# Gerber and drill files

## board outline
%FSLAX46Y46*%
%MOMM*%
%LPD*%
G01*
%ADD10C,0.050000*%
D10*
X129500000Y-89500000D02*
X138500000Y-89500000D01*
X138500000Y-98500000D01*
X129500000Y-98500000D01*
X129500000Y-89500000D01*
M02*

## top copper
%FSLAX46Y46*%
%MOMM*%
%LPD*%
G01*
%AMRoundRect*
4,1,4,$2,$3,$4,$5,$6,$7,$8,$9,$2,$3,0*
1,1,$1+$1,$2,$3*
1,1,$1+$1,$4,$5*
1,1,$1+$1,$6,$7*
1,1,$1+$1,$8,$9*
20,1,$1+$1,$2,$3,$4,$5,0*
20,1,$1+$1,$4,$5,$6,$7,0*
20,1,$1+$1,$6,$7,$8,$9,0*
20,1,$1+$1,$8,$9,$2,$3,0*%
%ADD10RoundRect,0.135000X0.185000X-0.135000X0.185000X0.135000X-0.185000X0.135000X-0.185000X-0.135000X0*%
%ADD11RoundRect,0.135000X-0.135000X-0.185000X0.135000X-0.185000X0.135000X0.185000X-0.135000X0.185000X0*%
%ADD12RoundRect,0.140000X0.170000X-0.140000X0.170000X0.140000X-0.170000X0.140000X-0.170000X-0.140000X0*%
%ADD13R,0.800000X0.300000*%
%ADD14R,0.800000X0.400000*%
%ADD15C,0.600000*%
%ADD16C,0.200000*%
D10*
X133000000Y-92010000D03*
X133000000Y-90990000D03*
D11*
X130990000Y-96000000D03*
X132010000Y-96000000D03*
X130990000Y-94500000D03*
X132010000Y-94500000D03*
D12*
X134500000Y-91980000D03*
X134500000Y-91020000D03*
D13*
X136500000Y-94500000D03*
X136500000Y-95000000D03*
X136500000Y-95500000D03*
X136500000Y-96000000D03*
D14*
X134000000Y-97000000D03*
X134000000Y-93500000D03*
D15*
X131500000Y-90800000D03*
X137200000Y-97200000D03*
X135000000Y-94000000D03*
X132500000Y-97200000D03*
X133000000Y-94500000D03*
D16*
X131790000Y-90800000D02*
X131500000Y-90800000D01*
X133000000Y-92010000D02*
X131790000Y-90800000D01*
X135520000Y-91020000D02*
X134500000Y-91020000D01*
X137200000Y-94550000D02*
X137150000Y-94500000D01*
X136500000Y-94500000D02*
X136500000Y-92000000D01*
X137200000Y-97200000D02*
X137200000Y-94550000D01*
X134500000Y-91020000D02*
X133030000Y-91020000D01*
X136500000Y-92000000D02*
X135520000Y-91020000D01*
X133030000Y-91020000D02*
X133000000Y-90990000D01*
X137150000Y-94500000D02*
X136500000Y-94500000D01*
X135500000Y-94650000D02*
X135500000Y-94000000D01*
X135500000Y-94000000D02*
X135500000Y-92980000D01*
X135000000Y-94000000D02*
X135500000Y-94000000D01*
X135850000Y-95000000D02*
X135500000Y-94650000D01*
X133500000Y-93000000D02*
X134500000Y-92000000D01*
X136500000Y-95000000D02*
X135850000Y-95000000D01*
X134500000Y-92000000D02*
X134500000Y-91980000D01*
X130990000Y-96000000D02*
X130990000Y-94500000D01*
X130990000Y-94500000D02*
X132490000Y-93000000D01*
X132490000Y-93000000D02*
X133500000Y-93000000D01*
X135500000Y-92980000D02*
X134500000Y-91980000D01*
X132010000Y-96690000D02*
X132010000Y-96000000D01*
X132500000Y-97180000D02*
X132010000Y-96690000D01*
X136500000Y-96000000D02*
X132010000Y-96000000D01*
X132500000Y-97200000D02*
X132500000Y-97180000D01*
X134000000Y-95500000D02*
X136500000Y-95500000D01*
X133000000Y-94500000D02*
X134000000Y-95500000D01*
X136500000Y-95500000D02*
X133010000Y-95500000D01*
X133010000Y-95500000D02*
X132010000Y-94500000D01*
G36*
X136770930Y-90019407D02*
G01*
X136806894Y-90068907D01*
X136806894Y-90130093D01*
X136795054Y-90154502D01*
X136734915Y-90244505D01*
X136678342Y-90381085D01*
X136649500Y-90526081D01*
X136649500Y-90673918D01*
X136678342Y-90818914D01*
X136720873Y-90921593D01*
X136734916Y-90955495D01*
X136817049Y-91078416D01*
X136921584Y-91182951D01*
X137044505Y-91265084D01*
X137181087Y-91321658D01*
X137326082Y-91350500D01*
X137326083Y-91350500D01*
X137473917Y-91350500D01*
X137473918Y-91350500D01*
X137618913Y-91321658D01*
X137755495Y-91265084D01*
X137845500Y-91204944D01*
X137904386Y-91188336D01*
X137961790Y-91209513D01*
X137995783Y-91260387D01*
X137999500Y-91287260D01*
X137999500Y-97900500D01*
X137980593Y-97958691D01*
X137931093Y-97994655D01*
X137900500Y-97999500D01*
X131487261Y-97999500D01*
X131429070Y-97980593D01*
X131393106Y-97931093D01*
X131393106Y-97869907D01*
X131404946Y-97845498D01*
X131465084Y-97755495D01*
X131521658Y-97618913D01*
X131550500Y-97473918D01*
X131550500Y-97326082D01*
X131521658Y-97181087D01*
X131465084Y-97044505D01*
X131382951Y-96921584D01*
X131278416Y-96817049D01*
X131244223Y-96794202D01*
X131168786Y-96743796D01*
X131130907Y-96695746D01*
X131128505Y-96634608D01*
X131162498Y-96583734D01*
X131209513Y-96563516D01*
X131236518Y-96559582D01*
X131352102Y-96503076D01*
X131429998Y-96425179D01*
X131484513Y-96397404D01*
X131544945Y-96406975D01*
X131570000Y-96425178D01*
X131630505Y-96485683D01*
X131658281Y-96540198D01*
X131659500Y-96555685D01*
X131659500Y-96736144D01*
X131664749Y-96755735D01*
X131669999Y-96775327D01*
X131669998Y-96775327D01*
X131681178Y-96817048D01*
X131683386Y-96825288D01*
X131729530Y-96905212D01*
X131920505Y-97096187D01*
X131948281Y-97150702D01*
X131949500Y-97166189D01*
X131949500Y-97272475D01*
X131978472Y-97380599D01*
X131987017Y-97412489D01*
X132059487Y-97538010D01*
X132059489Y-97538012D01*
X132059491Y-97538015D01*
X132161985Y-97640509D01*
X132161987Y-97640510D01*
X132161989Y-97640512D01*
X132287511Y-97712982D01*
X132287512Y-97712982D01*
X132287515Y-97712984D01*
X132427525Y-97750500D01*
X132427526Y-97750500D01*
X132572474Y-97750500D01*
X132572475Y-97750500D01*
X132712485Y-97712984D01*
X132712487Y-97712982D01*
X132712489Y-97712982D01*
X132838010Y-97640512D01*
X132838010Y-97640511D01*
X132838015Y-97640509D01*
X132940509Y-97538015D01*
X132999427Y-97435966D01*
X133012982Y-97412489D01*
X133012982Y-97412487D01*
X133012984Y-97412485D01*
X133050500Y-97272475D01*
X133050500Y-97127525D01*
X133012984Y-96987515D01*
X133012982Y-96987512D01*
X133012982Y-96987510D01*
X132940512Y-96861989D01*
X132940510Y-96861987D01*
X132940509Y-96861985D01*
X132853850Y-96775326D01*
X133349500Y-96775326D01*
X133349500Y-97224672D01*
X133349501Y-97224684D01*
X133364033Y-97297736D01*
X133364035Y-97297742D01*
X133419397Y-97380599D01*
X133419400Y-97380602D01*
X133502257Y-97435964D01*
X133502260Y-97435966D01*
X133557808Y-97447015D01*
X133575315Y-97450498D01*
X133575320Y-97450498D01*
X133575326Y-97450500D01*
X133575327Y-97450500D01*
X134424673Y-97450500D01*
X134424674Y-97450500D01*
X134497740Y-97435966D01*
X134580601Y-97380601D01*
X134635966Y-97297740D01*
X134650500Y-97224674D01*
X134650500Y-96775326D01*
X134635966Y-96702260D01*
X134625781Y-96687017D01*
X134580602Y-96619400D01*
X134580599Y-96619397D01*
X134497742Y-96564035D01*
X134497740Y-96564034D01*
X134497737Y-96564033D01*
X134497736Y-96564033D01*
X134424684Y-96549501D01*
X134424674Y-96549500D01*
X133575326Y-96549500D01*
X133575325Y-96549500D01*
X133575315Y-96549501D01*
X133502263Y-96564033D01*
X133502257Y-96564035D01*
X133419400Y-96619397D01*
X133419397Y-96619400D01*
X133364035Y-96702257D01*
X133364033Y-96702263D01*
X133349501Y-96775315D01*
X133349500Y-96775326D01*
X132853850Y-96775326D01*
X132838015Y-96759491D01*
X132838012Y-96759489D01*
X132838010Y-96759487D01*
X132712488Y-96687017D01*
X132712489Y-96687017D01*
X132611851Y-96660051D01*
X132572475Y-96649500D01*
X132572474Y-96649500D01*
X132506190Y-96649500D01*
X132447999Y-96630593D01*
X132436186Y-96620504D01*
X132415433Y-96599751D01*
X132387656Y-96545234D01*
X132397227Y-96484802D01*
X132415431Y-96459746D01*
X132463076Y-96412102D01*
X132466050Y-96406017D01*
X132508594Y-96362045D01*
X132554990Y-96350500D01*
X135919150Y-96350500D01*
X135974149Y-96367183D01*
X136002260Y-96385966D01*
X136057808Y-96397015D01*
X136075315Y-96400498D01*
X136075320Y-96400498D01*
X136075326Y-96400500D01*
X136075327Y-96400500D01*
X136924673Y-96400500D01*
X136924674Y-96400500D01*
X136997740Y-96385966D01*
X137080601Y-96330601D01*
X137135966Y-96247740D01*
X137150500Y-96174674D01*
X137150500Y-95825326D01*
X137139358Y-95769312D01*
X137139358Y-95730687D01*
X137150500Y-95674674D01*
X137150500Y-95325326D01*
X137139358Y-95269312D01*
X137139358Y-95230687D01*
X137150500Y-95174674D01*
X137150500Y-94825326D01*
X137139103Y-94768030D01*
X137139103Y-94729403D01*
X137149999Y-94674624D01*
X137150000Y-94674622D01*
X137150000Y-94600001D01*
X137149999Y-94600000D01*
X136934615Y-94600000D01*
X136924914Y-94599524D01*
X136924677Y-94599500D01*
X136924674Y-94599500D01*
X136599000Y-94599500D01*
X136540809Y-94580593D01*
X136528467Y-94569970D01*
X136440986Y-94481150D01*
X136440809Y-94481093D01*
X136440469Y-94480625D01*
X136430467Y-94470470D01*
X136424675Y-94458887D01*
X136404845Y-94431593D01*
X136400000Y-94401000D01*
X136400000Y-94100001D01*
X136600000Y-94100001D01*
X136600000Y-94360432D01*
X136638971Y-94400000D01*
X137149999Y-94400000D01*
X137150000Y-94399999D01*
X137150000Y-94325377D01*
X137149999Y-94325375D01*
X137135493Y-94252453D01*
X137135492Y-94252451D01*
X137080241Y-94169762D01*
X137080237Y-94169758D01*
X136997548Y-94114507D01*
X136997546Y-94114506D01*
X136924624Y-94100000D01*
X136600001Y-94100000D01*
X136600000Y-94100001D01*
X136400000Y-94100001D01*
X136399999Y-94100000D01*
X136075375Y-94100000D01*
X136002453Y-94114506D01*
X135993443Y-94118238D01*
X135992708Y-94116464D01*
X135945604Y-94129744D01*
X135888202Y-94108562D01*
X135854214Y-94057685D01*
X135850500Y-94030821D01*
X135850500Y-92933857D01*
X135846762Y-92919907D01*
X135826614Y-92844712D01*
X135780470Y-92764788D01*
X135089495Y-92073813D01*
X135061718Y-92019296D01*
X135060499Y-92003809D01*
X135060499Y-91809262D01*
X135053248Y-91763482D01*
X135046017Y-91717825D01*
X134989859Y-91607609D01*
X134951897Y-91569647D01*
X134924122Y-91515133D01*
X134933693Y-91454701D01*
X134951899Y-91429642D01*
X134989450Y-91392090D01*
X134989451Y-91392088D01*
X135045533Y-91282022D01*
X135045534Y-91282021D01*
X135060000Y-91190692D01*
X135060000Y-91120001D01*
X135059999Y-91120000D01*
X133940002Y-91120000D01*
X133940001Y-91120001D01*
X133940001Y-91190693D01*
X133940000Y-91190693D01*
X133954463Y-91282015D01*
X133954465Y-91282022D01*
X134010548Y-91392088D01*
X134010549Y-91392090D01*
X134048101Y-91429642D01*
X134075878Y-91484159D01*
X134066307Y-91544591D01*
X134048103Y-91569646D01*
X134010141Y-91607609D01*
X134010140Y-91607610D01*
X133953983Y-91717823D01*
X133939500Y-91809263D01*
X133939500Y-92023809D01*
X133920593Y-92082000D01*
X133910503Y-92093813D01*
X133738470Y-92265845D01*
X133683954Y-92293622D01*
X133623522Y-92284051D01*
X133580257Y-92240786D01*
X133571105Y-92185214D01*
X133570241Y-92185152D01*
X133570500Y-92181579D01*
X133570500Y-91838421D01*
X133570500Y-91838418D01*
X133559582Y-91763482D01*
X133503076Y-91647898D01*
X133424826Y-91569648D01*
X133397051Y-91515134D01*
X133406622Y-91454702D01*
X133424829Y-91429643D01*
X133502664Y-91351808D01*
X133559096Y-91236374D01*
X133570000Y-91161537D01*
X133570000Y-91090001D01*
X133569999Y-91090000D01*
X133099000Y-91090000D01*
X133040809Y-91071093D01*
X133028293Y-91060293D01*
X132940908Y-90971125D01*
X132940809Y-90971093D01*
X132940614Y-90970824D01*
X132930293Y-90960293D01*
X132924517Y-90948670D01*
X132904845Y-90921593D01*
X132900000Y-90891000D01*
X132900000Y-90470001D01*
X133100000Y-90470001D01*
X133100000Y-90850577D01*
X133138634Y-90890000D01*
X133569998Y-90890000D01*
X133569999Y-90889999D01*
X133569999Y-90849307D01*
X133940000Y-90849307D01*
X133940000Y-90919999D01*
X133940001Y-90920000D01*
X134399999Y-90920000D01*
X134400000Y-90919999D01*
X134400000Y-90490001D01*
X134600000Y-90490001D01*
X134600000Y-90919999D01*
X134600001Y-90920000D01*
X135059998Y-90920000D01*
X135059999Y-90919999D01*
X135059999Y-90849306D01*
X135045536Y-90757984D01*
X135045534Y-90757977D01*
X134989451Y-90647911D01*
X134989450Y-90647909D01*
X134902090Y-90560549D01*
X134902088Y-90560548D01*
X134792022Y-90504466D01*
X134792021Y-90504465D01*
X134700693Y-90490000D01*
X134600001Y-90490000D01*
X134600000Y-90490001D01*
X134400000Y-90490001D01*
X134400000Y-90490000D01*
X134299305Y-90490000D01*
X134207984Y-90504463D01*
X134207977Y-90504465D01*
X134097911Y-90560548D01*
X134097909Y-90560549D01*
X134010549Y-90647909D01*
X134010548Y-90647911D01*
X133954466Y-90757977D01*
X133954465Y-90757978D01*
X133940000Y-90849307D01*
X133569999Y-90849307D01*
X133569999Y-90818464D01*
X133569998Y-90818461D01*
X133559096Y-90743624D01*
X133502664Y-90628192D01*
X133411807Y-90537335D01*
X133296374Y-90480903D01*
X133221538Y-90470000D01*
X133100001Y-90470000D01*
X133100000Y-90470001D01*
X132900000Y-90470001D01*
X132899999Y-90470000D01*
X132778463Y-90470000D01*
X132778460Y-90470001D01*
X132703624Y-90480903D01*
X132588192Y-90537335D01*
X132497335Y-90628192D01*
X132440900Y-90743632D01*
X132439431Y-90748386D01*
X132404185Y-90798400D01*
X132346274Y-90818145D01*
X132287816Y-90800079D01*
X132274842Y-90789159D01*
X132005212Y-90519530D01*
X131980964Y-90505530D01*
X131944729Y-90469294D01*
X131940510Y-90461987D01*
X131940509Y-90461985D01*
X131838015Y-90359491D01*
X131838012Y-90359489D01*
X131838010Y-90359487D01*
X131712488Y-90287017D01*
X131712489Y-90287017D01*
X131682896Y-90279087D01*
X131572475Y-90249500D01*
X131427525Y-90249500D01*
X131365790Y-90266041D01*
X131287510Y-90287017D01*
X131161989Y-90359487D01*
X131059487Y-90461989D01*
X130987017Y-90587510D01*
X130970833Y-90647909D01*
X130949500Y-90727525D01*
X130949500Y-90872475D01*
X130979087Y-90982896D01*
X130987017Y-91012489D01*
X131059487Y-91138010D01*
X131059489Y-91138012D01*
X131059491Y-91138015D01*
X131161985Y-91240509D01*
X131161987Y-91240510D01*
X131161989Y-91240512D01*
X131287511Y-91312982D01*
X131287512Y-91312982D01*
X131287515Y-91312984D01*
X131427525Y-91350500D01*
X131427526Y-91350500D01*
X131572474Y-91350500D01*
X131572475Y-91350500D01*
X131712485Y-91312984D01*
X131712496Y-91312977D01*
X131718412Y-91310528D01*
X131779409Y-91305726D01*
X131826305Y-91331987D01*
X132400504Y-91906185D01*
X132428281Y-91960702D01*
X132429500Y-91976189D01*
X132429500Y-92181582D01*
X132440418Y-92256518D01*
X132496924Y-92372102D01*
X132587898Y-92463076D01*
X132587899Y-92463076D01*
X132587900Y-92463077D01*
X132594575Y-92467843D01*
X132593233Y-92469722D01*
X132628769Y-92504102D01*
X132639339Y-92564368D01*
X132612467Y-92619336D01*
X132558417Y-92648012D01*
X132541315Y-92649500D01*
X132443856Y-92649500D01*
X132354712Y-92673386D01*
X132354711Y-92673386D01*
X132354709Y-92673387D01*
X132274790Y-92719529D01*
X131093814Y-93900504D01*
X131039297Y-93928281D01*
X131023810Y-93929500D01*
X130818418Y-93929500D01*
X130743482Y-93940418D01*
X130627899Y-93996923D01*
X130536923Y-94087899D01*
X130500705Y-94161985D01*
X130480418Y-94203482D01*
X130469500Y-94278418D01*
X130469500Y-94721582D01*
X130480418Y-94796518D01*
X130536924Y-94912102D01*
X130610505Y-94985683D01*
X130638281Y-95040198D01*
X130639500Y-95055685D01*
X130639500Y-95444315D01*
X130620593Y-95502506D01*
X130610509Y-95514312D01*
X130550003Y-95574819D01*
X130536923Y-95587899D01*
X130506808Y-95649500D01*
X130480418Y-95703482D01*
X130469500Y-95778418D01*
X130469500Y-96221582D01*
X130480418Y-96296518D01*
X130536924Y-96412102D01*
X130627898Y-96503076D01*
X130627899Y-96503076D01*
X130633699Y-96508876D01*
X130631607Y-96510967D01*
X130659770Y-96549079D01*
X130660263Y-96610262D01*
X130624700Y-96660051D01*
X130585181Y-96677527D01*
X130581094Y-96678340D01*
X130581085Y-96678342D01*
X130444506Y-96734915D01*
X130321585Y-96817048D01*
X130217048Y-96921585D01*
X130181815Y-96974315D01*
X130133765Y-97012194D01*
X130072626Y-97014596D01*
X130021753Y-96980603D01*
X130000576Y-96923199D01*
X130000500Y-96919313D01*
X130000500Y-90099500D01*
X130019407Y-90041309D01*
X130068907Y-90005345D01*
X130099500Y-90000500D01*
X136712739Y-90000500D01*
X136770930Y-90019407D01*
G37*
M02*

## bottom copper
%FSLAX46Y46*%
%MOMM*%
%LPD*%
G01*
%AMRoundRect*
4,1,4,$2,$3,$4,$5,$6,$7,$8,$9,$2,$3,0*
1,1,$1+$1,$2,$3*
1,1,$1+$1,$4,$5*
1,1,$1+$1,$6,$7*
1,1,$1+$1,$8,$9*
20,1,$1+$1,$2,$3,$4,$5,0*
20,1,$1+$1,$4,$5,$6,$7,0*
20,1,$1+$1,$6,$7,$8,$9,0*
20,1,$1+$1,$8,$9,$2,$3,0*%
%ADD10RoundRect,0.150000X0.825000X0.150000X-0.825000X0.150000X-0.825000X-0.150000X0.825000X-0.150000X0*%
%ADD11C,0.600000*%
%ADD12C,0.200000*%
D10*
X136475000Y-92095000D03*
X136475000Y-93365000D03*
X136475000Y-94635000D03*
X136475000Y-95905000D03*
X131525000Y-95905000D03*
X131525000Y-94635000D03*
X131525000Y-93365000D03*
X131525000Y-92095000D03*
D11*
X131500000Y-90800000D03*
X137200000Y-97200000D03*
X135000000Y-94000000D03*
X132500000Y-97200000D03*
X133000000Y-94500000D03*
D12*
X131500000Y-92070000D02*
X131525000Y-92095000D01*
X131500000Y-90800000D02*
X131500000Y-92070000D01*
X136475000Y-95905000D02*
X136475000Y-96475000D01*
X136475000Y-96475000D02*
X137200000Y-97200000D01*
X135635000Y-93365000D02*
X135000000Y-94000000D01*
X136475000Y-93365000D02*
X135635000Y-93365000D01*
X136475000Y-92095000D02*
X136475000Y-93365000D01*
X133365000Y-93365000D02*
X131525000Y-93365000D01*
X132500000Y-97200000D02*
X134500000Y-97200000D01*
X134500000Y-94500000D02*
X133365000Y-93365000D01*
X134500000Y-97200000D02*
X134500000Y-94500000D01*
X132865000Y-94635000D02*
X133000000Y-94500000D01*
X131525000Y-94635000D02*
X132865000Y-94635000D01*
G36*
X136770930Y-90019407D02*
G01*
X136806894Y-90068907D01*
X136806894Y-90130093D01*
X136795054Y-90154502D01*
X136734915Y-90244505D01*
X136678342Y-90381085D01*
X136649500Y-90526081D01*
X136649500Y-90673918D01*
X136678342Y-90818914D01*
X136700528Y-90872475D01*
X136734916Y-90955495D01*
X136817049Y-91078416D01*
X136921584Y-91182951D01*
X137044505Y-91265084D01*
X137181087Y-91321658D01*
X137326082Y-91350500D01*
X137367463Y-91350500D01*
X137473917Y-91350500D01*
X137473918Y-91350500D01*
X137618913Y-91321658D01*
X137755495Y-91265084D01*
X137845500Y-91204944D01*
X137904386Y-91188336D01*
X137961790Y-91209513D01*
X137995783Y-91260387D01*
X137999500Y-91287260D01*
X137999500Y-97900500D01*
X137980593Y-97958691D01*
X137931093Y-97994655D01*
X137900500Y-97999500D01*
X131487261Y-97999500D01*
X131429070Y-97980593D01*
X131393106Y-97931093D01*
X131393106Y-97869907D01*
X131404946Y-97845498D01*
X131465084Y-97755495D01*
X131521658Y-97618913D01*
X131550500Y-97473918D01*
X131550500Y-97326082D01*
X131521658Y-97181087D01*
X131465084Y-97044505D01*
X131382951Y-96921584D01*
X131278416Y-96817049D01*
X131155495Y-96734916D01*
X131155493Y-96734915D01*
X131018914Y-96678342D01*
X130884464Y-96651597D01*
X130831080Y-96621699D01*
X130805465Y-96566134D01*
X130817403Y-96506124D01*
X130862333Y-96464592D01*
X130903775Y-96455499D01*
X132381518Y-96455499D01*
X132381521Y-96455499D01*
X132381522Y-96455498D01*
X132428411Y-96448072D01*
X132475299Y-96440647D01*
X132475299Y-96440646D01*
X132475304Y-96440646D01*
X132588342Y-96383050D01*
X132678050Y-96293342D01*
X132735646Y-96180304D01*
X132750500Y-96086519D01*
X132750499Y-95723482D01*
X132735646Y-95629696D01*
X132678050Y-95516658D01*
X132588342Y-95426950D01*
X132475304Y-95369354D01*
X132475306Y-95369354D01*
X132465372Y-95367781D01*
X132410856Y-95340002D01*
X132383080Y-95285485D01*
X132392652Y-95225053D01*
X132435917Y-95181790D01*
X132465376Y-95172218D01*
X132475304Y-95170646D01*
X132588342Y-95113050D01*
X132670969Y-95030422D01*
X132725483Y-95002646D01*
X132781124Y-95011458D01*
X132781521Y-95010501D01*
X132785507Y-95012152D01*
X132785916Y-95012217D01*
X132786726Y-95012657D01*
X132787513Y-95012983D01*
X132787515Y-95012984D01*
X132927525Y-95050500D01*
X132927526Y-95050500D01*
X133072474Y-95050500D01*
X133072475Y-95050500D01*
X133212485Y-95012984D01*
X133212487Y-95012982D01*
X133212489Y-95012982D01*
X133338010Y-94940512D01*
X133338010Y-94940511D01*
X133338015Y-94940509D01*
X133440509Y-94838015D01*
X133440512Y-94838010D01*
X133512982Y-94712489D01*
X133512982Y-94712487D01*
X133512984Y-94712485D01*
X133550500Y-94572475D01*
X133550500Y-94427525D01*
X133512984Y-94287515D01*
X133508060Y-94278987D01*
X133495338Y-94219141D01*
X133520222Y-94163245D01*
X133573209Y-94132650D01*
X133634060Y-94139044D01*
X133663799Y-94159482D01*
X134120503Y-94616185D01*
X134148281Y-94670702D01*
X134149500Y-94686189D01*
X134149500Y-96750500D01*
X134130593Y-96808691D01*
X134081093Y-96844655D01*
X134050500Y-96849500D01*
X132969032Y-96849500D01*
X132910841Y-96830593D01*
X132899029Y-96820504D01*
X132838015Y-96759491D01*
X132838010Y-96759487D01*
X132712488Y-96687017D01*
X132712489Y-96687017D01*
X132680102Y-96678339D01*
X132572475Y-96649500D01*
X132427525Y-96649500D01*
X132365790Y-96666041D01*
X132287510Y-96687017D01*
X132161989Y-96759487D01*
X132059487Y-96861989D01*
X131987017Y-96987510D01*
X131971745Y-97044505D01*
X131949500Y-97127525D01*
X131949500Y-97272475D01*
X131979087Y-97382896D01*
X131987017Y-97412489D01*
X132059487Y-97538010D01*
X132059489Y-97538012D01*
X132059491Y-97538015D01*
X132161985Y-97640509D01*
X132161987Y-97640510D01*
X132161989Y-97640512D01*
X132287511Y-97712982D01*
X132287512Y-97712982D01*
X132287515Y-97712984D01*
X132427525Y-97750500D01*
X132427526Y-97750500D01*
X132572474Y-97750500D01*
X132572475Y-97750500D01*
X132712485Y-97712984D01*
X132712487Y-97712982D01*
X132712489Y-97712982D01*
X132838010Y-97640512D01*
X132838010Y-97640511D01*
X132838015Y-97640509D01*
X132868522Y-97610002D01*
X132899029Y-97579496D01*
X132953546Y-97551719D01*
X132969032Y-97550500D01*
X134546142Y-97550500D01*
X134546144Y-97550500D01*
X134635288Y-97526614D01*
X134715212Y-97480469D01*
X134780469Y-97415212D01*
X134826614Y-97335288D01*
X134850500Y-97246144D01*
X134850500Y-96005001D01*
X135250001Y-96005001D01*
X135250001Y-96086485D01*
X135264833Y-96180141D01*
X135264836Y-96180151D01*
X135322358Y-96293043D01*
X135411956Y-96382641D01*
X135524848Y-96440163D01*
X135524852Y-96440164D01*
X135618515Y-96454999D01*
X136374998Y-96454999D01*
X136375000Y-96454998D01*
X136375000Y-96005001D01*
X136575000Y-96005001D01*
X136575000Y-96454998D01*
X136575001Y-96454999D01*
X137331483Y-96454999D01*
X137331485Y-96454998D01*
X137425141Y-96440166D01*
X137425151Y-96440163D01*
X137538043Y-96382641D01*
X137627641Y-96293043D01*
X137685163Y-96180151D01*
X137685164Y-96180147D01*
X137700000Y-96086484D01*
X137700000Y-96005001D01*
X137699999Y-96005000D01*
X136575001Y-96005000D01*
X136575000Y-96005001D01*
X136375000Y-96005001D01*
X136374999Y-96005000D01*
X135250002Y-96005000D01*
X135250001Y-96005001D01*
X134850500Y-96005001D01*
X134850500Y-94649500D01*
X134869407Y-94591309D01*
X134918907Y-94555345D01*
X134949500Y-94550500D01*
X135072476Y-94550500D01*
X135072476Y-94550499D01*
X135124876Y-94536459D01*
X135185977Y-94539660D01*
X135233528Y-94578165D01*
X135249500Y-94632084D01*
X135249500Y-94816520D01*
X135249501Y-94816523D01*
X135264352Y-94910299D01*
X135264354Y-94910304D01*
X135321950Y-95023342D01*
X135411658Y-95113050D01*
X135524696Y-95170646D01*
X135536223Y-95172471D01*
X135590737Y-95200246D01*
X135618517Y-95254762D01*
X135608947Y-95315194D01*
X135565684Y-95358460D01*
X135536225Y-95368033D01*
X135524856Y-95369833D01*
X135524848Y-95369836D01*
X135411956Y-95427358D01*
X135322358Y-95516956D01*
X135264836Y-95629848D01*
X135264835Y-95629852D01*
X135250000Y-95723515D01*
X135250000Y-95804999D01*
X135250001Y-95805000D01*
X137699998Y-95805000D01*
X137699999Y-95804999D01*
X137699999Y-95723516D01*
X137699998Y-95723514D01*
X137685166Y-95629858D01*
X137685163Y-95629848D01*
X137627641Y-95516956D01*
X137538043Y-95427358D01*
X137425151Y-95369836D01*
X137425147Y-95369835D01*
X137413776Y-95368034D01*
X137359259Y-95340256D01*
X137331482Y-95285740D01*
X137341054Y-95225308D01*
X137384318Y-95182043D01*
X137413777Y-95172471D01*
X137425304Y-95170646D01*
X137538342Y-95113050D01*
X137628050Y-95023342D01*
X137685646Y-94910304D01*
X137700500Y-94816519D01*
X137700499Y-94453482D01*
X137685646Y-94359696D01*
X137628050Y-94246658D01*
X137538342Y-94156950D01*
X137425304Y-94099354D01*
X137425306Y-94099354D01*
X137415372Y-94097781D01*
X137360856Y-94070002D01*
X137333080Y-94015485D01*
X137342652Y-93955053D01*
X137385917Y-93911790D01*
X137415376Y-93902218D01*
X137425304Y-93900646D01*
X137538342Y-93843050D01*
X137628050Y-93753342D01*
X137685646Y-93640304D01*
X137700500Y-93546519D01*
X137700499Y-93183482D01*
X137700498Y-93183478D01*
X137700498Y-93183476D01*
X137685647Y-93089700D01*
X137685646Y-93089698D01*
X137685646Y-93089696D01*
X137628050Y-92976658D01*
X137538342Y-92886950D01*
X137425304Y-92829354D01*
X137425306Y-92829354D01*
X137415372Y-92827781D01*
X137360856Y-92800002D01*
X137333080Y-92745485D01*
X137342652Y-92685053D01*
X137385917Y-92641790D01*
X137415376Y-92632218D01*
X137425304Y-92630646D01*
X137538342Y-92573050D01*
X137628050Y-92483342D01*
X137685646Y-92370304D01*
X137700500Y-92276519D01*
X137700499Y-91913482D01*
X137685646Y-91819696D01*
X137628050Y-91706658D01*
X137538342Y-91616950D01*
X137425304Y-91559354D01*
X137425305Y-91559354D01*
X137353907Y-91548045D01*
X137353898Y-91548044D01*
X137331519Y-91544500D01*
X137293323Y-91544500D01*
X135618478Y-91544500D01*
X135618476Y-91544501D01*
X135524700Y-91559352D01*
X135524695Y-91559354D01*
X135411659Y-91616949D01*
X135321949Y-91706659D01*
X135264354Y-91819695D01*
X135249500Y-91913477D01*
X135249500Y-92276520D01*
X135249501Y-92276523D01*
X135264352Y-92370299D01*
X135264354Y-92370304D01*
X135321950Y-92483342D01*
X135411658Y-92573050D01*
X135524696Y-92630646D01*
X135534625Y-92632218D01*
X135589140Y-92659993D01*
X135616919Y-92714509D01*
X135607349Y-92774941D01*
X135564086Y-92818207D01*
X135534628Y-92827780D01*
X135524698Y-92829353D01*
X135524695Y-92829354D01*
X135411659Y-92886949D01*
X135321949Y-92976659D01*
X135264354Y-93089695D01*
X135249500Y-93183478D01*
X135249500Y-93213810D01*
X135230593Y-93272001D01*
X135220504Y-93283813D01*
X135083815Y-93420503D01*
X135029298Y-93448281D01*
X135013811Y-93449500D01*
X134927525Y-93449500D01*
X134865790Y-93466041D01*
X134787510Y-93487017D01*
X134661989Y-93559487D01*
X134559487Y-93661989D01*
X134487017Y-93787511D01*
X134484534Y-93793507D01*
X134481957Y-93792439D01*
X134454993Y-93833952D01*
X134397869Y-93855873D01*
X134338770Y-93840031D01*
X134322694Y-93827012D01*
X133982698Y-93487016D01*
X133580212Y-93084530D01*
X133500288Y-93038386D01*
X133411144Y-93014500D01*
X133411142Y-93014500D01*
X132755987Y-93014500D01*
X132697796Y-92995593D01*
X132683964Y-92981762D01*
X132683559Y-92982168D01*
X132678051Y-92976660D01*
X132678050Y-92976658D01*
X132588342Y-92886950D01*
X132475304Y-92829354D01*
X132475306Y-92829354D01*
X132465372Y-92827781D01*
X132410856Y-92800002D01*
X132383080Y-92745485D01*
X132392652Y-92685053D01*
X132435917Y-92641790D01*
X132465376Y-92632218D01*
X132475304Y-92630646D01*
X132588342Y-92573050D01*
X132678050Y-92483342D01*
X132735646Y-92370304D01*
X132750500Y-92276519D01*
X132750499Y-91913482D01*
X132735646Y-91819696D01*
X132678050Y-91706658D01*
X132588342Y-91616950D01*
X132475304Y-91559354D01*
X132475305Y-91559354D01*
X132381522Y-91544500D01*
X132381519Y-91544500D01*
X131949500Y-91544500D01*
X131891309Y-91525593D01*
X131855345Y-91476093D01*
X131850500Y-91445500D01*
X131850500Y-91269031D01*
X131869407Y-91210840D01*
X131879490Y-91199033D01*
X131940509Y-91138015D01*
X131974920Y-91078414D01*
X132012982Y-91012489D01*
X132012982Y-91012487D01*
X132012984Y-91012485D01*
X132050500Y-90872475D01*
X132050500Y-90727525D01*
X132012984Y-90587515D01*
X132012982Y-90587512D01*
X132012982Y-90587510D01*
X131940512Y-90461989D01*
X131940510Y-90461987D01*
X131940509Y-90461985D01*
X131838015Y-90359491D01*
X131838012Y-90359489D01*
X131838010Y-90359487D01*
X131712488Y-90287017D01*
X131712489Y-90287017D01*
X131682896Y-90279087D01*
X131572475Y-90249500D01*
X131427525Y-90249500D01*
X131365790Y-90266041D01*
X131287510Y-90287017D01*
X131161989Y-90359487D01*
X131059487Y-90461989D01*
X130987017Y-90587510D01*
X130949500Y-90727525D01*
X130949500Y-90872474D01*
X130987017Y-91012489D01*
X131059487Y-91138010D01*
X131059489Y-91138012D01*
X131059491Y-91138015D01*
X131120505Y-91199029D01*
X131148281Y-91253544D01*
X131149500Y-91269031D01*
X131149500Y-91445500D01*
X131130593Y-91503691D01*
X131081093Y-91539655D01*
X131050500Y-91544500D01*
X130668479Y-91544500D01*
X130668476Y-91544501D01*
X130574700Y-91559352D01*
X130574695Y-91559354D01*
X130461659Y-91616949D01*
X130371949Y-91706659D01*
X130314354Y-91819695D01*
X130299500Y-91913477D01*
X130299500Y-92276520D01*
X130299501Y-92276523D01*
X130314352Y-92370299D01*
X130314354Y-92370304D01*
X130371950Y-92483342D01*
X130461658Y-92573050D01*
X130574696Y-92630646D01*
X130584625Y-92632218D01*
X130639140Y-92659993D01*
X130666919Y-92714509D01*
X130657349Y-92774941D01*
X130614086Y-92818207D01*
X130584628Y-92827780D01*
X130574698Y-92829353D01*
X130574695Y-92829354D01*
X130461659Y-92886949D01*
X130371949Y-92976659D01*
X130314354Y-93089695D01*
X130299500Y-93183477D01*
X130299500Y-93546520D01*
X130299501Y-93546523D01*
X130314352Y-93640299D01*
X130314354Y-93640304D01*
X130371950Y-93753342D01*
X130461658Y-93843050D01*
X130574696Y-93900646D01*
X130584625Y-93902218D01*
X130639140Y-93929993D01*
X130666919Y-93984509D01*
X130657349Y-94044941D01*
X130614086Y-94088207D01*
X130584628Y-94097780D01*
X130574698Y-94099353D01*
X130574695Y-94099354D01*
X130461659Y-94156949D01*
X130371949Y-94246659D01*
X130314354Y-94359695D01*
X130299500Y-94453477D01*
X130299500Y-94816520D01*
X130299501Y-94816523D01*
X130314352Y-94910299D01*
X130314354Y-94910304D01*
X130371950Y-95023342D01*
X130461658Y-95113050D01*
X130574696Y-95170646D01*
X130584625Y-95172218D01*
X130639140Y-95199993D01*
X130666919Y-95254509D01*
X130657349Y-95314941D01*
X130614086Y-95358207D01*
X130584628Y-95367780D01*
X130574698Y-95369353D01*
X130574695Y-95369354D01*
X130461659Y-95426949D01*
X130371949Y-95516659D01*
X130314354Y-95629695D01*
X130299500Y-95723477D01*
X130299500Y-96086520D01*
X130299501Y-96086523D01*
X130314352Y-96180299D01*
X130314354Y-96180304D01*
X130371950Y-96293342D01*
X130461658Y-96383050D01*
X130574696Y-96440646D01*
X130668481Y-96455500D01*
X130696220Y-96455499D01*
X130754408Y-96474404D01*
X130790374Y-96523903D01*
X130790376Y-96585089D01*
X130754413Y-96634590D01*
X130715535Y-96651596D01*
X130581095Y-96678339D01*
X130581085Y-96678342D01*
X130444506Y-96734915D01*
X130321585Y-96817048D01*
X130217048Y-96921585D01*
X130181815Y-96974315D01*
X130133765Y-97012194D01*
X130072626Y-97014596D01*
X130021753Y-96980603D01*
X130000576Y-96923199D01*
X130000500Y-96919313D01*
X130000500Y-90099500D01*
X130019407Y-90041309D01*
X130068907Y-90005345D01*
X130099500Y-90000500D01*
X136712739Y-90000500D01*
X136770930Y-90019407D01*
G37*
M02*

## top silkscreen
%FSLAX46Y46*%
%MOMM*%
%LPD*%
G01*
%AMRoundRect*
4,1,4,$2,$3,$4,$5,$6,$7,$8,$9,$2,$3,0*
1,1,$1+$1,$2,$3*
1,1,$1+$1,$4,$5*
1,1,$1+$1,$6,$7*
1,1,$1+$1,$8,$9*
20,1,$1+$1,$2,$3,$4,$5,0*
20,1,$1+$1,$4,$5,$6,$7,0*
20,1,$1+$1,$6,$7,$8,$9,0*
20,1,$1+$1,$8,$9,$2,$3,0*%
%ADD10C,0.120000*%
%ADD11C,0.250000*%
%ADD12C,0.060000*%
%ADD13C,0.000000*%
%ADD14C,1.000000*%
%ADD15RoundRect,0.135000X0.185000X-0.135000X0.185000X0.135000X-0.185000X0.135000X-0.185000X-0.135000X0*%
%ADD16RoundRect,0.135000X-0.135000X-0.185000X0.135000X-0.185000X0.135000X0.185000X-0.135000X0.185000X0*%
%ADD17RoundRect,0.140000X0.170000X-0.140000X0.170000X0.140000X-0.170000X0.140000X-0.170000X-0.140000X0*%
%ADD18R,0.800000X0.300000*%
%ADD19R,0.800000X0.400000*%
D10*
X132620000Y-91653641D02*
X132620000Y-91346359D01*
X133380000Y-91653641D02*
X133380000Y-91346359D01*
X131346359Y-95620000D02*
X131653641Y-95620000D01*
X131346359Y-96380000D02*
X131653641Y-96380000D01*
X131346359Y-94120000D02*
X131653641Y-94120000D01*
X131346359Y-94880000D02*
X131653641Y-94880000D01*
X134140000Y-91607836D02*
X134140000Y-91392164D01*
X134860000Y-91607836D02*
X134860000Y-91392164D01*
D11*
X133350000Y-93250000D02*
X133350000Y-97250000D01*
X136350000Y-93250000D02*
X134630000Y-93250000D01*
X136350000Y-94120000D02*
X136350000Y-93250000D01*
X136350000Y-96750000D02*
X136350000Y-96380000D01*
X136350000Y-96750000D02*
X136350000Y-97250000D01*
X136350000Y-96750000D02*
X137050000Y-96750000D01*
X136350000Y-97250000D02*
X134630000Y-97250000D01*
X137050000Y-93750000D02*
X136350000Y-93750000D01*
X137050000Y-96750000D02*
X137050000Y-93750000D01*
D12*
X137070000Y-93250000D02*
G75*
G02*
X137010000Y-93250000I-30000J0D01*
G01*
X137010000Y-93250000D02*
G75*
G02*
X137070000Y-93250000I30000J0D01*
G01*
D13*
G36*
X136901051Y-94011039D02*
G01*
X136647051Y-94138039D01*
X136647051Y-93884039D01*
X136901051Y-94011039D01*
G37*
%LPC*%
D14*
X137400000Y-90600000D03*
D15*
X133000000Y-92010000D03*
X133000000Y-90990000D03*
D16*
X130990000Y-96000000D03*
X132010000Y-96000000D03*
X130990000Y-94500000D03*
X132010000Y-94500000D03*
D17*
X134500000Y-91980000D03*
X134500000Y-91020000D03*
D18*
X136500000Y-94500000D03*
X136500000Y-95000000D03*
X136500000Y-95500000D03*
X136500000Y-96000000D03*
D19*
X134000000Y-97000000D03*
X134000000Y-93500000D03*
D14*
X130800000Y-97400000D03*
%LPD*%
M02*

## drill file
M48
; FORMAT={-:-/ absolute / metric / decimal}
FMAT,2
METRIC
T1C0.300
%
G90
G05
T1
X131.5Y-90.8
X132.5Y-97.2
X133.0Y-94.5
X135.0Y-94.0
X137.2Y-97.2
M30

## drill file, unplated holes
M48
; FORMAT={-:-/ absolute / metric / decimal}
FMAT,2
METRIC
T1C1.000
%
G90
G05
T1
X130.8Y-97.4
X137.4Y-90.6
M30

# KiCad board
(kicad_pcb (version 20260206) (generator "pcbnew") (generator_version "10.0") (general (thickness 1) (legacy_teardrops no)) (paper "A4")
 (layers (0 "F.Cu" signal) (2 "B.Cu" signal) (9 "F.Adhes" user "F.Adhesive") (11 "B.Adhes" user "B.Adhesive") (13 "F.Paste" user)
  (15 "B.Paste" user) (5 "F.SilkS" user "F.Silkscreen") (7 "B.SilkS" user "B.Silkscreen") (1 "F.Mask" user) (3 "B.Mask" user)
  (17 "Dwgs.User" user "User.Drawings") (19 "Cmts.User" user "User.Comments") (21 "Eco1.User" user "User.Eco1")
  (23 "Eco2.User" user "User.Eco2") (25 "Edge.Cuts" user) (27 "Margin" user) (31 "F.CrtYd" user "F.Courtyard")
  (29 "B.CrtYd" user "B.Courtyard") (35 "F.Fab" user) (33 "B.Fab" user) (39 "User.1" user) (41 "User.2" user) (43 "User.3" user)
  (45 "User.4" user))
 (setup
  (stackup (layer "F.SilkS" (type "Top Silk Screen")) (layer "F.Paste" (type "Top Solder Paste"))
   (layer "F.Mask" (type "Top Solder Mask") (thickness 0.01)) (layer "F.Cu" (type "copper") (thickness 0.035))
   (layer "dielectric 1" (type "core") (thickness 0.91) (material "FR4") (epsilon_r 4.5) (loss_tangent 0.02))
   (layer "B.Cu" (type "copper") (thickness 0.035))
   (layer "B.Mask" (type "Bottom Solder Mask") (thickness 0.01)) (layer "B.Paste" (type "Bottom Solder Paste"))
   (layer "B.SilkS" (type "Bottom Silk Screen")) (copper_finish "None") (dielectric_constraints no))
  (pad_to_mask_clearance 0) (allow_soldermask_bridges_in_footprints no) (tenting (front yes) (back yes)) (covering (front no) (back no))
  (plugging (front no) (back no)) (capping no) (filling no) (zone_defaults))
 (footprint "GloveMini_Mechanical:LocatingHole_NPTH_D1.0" (layer "F.Cu") (at 137.4 90.6)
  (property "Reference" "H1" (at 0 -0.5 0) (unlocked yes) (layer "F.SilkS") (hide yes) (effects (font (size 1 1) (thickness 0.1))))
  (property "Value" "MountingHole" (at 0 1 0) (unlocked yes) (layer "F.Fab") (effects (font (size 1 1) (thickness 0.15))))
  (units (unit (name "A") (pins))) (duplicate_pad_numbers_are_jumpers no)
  (pad "" np_thru_hole circle (at 0 0) (size 1 1) (drill 1) (layers "*.Cu" "*.Mask")))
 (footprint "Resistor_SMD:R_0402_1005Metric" (layer "F.Cu") (at 133 91.5 90)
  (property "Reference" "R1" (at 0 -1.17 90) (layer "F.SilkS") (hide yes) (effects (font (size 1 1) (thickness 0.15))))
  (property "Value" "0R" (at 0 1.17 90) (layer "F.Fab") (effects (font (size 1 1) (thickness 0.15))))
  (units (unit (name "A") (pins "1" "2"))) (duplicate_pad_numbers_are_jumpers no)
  (fp_line (start -0.153641 -0.38) (end 0.153641 -0.38) (stroke (width 0.12) (type solid)) (layer "F.SilkS"))
  (fp_line (start -0.153641 0.38) (end 0.153641 0.38) (stroke (width 0.12) (type solid)) (layer "F.SilkS"))
  (pad "1" smd roundrect (at -0.51 0 90) (size 0.54 0.64) (layers "F.Cu" "F.Mask" "F.Paste") (roundrect_rratio 0.25) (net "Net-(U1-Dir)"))
  (pad "2" smd roundrect (at 0.51 0 90) (size 0.54 0.64) (layers "F.Cu" "F.Mask" "F.Paste") (roundrect_rratio 0.25) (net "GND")))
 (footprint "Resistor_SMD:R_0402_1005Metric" (layer "F.Cu") (at 131.5 96)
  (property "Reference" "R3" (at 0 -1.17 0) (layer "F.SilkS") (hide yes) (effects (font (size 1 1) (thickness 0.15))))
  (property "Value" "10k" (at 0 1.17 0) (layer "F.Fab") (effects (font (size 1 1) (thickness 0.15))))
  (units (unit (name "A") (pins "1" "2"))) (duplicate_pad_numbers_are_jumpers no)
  (fp_line (start -0.153641 -0.38) (end 0.153641 -0.38) (stroke (width 0.12) (type solid)) (layer "F.SilkS"))
  (fp_line (start -0.153641 0.38) (end 0.153641 0.38) (stroke (width 0.12) (type solid)) (layer "F.SilkS"))
  (pad "1" smd roundrect (at -0.51 0) (size 0.54 0.64) (layers "F.Cu" "F.Mask" "F.Paste") (roundrect_rratio 0.25) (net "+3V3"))
  (pad "2" smd roundrect (at 0.51 0) (size 0.54 0.64) (layers "F.Cu" "F.Mask" "F.Paste") (roundrect_rratio 0.25) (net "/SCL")))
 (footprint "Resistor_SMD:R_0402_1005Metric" (layer "F.Cu") (at 131.5 94.5)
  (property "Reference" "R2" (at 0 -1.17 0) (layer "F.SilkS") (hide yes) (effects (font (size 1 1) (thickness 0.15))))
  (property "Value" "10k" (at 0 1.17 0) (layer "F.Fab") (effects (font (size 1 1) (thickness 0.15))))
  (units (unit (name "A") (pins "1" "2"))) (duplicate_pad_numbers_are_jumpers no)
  (fp_line (start -0.153641 -0.38) (end 0.153641 -0.38) (stroke (width 0.12) (type solid)) (layer "F.SilkS"))
  (fp_line (start -0.153641 0.38) (end 0.153641 0.38) (stroke (width 0.12) (type solid)) (layer "F.SilkS"))
  (pad "1" smd roundrect (at -0.51 0) (size 0.54 0.64) (layers "F.Cu" "F.Mask" "F.Paste") (roundrect_rratio 0.25) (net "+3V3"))
  (pad "2" smd roundrect (at 0.51 0) (size 0.54 0.64) (layers "F.Cu" "F.Mask" "F.Paste") (roundrect_rratio 0.25) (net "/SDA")))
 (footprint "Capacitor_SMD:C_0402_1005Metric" (layer "F.Cu") (at 134.5 91.5 90)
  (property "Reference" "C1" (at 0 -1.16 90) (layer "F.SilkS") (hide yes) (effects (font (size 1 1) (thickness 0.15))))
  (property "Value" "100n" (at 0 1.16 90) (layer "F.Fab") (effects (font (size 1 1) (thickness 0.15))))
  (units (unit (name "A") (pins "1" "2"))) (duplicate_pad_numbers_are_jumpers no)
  (fp_line (start -0.107836 -0.36) (end 0.107836 -0.36) (stroke (width 0.12) (type solid)) (layer "F.SilkS"))
  (fp_line (start -0.107836 0.36) (end 0.107836 0.36) (stroke (width 0.12) (type solid)) (layer "F.SilkS"))
  (pad "1" smd roundrect (at -0.48 0 90) (size 0.56 0.62) (layers "F.Cu" "F.Mask" "F.Paste") (roundrect_rratio 0.25) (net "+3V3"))
  (pad "2" smd roundrect (at 0.48 0 90) (size 0.56 0.62) (layers "F.Cu" "F.Mask" "F.Paste") (roundrect_rratio 0.25) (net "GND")))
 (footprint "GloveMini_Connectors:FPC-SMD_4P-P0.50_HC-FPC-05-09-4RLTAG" (layer "F.Cu") (at 135.25 95.25 90)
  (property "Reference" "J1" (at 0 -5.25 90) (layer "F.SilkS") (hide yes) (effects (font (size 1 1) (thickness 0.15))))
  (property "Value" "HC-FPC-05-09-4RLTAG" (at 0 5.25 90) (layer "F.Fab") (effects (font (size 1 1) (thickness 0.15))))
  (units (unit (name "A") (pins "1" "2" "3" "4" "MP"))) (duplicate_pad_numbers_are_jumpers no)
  (fp_line (start 2 -1.9) (end -2 -1.9) (stroke (width 0.25) (type solid)) (layer "F.SilkS"))
  (fp_line (start 2 1.1) (end 2 -0.62) (stroke (width 0.25) (type solid)) (layer "F.SilkS"))
  (fp_line (start 1.13 1.1) (end 2 1.1) (stroke (width 0.25) (type solid)) (layer "F.SilkS"))
  (fp_line (start -1.5 1.1) (end -1.13 1.1) (stroke (width 0.25) (type solid)) (layer "F.SilkS"))
  (fp_line (start -1.5 1.1) (end -2 1.1) (stroke (width 0.25) (type solid)) (layer "F.SilkS"))
  (fp_line (start -1.5 1.1) (end -1.5 1.8) (stroke (width 0.25) (type solid)) (layer "F.SilkS"))
  (fp_line (start -2 1.1) (end -2 -0.62) (stroke (width 0.25) (type solid)) (layer "F.SilkS"))
  (fp_line (start 1.5 1.8) (end 1.5 1.1) (stroke (width 0.25) (type solid)) (layer "F.SilkS"))
  (fp_line (start -1.5 1.8) (end 1.5 1.8) (stroke (width 0.25) (type solid)) (layer "F.SilkS"))
  (fp_circle (center 2 1.79) (end 2.03 1.79) (stroke (width 0.06) (type solid)) (fill no) (layer "F.SilkS"))
  (fp_poly
   (pts (xy 1.238961 1.651051) (xy 1.365961 1.397051) (xy 1.238961 1.524051) (xy 1.365961 1.397051) (xy 1.111961 1.397051)
    (xy 1.238961 1.651051))
   (stroke (width 0) (type solid)) (fill yes) (layer "F.SilkS"))
  (pad "1" smd rect (at 0.75 1.25 270) (size 0.3 0.8) (layers "F.Cu" "F.Mask" "F.Paste") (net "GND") (solder_paste_margin 0.005)
   (solder_paste_margin_ratio -0.1))
  (pad "2" smd rect (at 0.25 1.25 270) (size 0.3 0.8) (layers "F.Cu" "F.Mask" "F.Paste") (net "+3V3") (solder_paste_margin 0.005)
   (solder_paste_margin_ratio -0.1))
  (pad "3" smd rect (at -0.25 1.25 270) (size 0.3 0.8) (layers "F.Cu" "F.Mask" "F.Paste") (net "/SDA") (solder_paste_margin 0.005)
   (solder_paste_margin_ratio -0.1))
  (pad "4" smd rect (at -0.75 1.25 270) (size 0.3 0.8) (layers "F.Cu" "F.Mask" "F.Paste") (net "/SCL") (solder_paste_margin 0.005)
   (solder_paste_margin_ratio -0.1))
  (pad "MP" smd rect (at -1.75 -1.25 270) (size 0.4 0.8) (layers "F.Cu" "F.Mask" "F.Paste") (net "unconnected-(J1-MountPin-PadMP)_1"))
  (pad "MP" smd rect (at 1.75 -1.25 270) (size 0.4 0.8) (layers "F.Cu" "F.Mask" "F.Paste") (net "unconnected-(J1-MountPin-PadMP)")))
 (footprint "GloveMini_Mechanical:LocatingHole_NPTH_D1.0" (layer "F.Cu") (at 130.8 97.4)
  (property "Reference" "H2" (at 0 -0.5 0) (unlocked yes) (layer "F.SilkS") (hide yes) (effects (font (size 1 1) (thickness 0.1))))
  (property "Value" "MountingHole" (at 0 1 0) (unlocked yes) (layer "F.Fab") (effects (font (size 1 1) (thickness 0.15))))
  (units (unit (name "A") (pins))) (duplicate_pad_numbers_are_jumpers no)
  (pad "" np_thru_hole circle (at 0 0) (size 1 1) (drill 1) (layers "*.Cu" "*.Mask")))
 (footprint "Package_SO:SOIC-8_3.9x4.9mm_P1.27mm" (layer "B.Cu") (at 134 94 180)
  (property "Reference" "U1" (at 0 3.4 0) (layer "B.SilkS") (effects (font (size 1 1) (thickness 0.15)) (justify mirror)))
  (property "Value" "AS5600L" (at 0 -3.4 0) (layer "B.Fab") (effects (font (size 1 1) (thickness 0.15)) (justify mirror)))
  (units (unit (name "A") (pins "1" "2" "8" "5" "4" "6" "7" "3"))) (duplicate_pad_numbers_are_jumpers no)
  (pad "1" smd roundrect (at -2.475 1.905 180) (size 1.95 0.6) (layers "B.Cu" "B.Mask" "B.Paste") (roundrect_rratio 0.25) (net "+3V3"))
  (pad "2" smd roundrect (at -2.475 0.635 180) (size 1.95 0.6) (layers "B.Cu" "B.Mask" "B.Paste") (roundrect_rratio 0.25) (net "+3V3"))
  (pad "3" smd roundrect (at -2.475 -0.635 180) (size 1.95 0.6) (layers "B.Cu" "B.Mask" "B.Paste") (roundrect_rratio 0.25)
   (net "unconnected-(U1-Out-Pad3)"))
  (pad "4" smd roundrect (at -2.475 -1.905 180) (size 1.95 0.6) (layers "B.Cu" "B.Mask" "B.Paste") (roundrect_rratio 0.25) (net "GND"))
  (pad "5" smd roundrect (at 2.475 -1.905 180) (size 1.95 0.6) (layers "B.Cu" "B.Mask" "B.Paste") (roundrect_rratio 0.25)
   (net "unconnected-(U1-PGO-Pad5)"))
  (pad "6" smd roundrect (at 2.475 -0.635 180) (size 1.95 0.6) (layers "B.Cu" "B.Mask" "B.Paste") (roundrect_rratio 0.25) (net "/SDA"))
  (pad "7" smd roundrect (at 2.475 0.635 180) (size 1.95 0.6) (layers "B.Cu" "B.Mask" "B.Paste") (roundrect_rratio 0.25) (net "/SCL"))
  (pad "8" smd roundrect (at 2.475 1.905 180) (size 1.95 0.6) (layers "B.Cu" "B.Mask" "B.Paste") (roundrect_rratio 0.25)
   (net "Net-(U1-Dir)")))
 (gr_rect (start 129.5 89.5) (end 138.5 98.5) (stroke (width 0.05) (type solid)) (fill no) (layer "Edge.Cuts"))
 (segment (start 131.79 90.8) (end 131.5 90.8) (width 0.2) (layer "F.Cu") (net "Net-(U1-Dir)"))
 (segment (start 133 92.01) (end 131.79 90.8) (width 0.2) (layer "F.Cu") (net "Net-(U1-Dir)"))
 (via (at 131.5 90.8) (size 0.6) (drill 0.3) (layers "F.Cu" "B.Cu") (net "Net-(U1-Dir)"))
 (segment (start 131.5 92.07) (end 131.525 92.095) (width 0.2) (layer "B.Cu") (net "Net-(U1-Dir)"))
 (segment (start 131.5 90.8) (end 131.5 92.07) (width 0.2) (layer "B.Cu") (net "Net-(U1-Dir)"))
 (segment (start 135.52 91.02) (end 134.5 91.02) (width 0.2) (layer "F.Cu") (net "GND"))
 (segment (start 137.2 94.55) (end 137.15 94.5) (width 0.2) (layer "F.Cu") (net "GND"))
 (segment (start 136.5 94.5) (end 136.5 92) (width 0.2) (layer "F.Cu") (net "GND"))
 (segment (start 137.2 97.2) (end 137.2 94.55) (width 0.2) (layer "F.Cu") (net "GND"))
 (segment (start 134.5 91.02) (end 133.03 91.02) (width 0.2) (layer "F.Cu") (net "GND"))
 (segment (start 136.5 92) (end 135.52 91.02) (width 0.2) (layer "F.Cu") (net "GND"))
 (segment (start 133.03 91.02) (end 133 90.99) (width 0.2) (layer "F.Cu") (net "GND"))
 (segment (start 137.15 94.5) (end 136.5 94.5) (width 0.2) (layer "F.Cu") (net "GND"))
 (via (at 137.2 97.2) (size 0.6) (drill 0.3) (layers "F.Cu" "B.Cu") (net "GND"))
 (segment (start 136.475 95.905) (end 136.475 96.475) (width 0.2) (layer "B.Cu") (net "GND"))
 (segment (start 136.475 96.475) (end 137.2 97.2) (width 0.2) (layer "B.Cu") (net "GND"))
 (segment (start 135.5 94.65) (end 135.5 94) (width 0.2) (layer "F.Cu") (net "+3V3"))
 (segment (start 135.5 94) (end 135.5 92.98) (width 0.2) (layer "F.Cu") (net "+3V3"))
 (segment (start 135 94) (end 135.5 94) (width 0.2) (layer "F.Cu") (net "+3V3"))
 (segment (start 135.85 95) (end 135.5 94.65) (width 0.2) (layer "F.Cu") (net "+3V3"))
 (segment (start 133.5 93) (end 134.5 92) (width 0.2) (layer "F.Cu") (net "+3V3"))
 (segment (start 136.5 95) (end 135.85 95) (width 0.2) (layer "F.Cu") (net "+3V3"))
 (segment (start 134.5 92) (end 134.5 91.98) (width 0.2) (layer "F.Cu") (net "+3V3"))
 (segment (start 130.99 96) (end 130.99 94.5) (width 0.2) (layer "F.Cu") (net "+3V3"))
 (segment (start 130.99 94.5) (end 132.49 93) (width 0.2) (layer "F.Cu") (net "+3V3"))
 (segment (start 132.49 93) (end 133.5 93) (width 0.2) (layer "F.Cu") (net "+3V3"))
 (segment (start 135.5 92.98) (end 134.5 91.98) (width 0.2) (layer "F.Cu") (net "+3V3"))
 (via (at 135 94) (size 0.6) (drill 0.3) (layers "F.Cu" "B.Cu") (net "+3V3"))
 (segment (start 135.635 93.365) (end 135 94) (width 0.2) (layer "B.Cu") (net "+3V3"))
 (segment (start 136.475 93.365) (end 135.635 93.365) (width 0.2) (layer "B.Cu") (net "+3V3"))
 (segment (start 136.475 92.095) (end 136.475 93.365) (width 0.2) (layer "B.Cu") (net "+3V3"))
 (segment (start 132.01 96.69) (end 132.01 96) (width 0.2) (layer "F.Cu") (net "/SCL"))
 (segment (start 132.5 97.18) (end 132.01 96.69) (width 0.2) (layer "F.Cu") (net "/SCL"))
 (segment (start 136.5 96) (end 132.01 96) (width 0.2) (layer "F.Cu") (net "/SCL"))
 (segment (start 132.5 97.2) (end 132.5 97.18) (width 0.2) (layer "F.Cu") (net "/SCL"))
 (via (at 132.5 97.2) (size 0.6) (drill 0.3) (layers "F.Cu" "B.Cu") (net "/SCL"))
 (segment (start 133.365 93.365) (end 131.525 93.365) (width 0.2) (layer "B.Cu") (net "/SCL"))
 (segment (start 132.5 97.2) (end 134.5 97.2) (width 0.2) (layer "B.Cu") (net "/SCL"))
 (segment (start 134.5 94.5) (end 133.365 93.365) (width 0.2) (layer "B.Cu") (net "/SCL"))
 (segment (start 134.5 97.2) (end 134.5 94.5) (width 0.2) (layer "B.Cu") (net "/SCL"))
 (segment (start 134 95.5) (end 136.5 95.5) (width 0.2) (layer "F.Cu") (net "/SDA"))
 (segment (start 133 94.5) (end 134 95.5) (width 0.2) (layer "F.Cu") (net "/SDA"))
 (segment (start 136.5 95.5) (end 133.01 95.5) (width 0.2) (layer "F.Cu") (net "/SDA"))
 (segment (start 133.01 95.5) (end 132.01 94.5) (width 0.2) (layer "F.Cu") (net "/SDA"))
 (via (at 133 94.5) (size 0.6) (drill 0.3) (layers "F.Cu" "B.Cu") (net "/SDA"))
 (segment (start 132.865 94.635) (end 133 94.5) (width 0.2) (layer "B.Cu") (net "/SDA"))
 (segment (start 131.525 94.635) (end 132.865 94.635) (width 0.2) (layer "B.Cu") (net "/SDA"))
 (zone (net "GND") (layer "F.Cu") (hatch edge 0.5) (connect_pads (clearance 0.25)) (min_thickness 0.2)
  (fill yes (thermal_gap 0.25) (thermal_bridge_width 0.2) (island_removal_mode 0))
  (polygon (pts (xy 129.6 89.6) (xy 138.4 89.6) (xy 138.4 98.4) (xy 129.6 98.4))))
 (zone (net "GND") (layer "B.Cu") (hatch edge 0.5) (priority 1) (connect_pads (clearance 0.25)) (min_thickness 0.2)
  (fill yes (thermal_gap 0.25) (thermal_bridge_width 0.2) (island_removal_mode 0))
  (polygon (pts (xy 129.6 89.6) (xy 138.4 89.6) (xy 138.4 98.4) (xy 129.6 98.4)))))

